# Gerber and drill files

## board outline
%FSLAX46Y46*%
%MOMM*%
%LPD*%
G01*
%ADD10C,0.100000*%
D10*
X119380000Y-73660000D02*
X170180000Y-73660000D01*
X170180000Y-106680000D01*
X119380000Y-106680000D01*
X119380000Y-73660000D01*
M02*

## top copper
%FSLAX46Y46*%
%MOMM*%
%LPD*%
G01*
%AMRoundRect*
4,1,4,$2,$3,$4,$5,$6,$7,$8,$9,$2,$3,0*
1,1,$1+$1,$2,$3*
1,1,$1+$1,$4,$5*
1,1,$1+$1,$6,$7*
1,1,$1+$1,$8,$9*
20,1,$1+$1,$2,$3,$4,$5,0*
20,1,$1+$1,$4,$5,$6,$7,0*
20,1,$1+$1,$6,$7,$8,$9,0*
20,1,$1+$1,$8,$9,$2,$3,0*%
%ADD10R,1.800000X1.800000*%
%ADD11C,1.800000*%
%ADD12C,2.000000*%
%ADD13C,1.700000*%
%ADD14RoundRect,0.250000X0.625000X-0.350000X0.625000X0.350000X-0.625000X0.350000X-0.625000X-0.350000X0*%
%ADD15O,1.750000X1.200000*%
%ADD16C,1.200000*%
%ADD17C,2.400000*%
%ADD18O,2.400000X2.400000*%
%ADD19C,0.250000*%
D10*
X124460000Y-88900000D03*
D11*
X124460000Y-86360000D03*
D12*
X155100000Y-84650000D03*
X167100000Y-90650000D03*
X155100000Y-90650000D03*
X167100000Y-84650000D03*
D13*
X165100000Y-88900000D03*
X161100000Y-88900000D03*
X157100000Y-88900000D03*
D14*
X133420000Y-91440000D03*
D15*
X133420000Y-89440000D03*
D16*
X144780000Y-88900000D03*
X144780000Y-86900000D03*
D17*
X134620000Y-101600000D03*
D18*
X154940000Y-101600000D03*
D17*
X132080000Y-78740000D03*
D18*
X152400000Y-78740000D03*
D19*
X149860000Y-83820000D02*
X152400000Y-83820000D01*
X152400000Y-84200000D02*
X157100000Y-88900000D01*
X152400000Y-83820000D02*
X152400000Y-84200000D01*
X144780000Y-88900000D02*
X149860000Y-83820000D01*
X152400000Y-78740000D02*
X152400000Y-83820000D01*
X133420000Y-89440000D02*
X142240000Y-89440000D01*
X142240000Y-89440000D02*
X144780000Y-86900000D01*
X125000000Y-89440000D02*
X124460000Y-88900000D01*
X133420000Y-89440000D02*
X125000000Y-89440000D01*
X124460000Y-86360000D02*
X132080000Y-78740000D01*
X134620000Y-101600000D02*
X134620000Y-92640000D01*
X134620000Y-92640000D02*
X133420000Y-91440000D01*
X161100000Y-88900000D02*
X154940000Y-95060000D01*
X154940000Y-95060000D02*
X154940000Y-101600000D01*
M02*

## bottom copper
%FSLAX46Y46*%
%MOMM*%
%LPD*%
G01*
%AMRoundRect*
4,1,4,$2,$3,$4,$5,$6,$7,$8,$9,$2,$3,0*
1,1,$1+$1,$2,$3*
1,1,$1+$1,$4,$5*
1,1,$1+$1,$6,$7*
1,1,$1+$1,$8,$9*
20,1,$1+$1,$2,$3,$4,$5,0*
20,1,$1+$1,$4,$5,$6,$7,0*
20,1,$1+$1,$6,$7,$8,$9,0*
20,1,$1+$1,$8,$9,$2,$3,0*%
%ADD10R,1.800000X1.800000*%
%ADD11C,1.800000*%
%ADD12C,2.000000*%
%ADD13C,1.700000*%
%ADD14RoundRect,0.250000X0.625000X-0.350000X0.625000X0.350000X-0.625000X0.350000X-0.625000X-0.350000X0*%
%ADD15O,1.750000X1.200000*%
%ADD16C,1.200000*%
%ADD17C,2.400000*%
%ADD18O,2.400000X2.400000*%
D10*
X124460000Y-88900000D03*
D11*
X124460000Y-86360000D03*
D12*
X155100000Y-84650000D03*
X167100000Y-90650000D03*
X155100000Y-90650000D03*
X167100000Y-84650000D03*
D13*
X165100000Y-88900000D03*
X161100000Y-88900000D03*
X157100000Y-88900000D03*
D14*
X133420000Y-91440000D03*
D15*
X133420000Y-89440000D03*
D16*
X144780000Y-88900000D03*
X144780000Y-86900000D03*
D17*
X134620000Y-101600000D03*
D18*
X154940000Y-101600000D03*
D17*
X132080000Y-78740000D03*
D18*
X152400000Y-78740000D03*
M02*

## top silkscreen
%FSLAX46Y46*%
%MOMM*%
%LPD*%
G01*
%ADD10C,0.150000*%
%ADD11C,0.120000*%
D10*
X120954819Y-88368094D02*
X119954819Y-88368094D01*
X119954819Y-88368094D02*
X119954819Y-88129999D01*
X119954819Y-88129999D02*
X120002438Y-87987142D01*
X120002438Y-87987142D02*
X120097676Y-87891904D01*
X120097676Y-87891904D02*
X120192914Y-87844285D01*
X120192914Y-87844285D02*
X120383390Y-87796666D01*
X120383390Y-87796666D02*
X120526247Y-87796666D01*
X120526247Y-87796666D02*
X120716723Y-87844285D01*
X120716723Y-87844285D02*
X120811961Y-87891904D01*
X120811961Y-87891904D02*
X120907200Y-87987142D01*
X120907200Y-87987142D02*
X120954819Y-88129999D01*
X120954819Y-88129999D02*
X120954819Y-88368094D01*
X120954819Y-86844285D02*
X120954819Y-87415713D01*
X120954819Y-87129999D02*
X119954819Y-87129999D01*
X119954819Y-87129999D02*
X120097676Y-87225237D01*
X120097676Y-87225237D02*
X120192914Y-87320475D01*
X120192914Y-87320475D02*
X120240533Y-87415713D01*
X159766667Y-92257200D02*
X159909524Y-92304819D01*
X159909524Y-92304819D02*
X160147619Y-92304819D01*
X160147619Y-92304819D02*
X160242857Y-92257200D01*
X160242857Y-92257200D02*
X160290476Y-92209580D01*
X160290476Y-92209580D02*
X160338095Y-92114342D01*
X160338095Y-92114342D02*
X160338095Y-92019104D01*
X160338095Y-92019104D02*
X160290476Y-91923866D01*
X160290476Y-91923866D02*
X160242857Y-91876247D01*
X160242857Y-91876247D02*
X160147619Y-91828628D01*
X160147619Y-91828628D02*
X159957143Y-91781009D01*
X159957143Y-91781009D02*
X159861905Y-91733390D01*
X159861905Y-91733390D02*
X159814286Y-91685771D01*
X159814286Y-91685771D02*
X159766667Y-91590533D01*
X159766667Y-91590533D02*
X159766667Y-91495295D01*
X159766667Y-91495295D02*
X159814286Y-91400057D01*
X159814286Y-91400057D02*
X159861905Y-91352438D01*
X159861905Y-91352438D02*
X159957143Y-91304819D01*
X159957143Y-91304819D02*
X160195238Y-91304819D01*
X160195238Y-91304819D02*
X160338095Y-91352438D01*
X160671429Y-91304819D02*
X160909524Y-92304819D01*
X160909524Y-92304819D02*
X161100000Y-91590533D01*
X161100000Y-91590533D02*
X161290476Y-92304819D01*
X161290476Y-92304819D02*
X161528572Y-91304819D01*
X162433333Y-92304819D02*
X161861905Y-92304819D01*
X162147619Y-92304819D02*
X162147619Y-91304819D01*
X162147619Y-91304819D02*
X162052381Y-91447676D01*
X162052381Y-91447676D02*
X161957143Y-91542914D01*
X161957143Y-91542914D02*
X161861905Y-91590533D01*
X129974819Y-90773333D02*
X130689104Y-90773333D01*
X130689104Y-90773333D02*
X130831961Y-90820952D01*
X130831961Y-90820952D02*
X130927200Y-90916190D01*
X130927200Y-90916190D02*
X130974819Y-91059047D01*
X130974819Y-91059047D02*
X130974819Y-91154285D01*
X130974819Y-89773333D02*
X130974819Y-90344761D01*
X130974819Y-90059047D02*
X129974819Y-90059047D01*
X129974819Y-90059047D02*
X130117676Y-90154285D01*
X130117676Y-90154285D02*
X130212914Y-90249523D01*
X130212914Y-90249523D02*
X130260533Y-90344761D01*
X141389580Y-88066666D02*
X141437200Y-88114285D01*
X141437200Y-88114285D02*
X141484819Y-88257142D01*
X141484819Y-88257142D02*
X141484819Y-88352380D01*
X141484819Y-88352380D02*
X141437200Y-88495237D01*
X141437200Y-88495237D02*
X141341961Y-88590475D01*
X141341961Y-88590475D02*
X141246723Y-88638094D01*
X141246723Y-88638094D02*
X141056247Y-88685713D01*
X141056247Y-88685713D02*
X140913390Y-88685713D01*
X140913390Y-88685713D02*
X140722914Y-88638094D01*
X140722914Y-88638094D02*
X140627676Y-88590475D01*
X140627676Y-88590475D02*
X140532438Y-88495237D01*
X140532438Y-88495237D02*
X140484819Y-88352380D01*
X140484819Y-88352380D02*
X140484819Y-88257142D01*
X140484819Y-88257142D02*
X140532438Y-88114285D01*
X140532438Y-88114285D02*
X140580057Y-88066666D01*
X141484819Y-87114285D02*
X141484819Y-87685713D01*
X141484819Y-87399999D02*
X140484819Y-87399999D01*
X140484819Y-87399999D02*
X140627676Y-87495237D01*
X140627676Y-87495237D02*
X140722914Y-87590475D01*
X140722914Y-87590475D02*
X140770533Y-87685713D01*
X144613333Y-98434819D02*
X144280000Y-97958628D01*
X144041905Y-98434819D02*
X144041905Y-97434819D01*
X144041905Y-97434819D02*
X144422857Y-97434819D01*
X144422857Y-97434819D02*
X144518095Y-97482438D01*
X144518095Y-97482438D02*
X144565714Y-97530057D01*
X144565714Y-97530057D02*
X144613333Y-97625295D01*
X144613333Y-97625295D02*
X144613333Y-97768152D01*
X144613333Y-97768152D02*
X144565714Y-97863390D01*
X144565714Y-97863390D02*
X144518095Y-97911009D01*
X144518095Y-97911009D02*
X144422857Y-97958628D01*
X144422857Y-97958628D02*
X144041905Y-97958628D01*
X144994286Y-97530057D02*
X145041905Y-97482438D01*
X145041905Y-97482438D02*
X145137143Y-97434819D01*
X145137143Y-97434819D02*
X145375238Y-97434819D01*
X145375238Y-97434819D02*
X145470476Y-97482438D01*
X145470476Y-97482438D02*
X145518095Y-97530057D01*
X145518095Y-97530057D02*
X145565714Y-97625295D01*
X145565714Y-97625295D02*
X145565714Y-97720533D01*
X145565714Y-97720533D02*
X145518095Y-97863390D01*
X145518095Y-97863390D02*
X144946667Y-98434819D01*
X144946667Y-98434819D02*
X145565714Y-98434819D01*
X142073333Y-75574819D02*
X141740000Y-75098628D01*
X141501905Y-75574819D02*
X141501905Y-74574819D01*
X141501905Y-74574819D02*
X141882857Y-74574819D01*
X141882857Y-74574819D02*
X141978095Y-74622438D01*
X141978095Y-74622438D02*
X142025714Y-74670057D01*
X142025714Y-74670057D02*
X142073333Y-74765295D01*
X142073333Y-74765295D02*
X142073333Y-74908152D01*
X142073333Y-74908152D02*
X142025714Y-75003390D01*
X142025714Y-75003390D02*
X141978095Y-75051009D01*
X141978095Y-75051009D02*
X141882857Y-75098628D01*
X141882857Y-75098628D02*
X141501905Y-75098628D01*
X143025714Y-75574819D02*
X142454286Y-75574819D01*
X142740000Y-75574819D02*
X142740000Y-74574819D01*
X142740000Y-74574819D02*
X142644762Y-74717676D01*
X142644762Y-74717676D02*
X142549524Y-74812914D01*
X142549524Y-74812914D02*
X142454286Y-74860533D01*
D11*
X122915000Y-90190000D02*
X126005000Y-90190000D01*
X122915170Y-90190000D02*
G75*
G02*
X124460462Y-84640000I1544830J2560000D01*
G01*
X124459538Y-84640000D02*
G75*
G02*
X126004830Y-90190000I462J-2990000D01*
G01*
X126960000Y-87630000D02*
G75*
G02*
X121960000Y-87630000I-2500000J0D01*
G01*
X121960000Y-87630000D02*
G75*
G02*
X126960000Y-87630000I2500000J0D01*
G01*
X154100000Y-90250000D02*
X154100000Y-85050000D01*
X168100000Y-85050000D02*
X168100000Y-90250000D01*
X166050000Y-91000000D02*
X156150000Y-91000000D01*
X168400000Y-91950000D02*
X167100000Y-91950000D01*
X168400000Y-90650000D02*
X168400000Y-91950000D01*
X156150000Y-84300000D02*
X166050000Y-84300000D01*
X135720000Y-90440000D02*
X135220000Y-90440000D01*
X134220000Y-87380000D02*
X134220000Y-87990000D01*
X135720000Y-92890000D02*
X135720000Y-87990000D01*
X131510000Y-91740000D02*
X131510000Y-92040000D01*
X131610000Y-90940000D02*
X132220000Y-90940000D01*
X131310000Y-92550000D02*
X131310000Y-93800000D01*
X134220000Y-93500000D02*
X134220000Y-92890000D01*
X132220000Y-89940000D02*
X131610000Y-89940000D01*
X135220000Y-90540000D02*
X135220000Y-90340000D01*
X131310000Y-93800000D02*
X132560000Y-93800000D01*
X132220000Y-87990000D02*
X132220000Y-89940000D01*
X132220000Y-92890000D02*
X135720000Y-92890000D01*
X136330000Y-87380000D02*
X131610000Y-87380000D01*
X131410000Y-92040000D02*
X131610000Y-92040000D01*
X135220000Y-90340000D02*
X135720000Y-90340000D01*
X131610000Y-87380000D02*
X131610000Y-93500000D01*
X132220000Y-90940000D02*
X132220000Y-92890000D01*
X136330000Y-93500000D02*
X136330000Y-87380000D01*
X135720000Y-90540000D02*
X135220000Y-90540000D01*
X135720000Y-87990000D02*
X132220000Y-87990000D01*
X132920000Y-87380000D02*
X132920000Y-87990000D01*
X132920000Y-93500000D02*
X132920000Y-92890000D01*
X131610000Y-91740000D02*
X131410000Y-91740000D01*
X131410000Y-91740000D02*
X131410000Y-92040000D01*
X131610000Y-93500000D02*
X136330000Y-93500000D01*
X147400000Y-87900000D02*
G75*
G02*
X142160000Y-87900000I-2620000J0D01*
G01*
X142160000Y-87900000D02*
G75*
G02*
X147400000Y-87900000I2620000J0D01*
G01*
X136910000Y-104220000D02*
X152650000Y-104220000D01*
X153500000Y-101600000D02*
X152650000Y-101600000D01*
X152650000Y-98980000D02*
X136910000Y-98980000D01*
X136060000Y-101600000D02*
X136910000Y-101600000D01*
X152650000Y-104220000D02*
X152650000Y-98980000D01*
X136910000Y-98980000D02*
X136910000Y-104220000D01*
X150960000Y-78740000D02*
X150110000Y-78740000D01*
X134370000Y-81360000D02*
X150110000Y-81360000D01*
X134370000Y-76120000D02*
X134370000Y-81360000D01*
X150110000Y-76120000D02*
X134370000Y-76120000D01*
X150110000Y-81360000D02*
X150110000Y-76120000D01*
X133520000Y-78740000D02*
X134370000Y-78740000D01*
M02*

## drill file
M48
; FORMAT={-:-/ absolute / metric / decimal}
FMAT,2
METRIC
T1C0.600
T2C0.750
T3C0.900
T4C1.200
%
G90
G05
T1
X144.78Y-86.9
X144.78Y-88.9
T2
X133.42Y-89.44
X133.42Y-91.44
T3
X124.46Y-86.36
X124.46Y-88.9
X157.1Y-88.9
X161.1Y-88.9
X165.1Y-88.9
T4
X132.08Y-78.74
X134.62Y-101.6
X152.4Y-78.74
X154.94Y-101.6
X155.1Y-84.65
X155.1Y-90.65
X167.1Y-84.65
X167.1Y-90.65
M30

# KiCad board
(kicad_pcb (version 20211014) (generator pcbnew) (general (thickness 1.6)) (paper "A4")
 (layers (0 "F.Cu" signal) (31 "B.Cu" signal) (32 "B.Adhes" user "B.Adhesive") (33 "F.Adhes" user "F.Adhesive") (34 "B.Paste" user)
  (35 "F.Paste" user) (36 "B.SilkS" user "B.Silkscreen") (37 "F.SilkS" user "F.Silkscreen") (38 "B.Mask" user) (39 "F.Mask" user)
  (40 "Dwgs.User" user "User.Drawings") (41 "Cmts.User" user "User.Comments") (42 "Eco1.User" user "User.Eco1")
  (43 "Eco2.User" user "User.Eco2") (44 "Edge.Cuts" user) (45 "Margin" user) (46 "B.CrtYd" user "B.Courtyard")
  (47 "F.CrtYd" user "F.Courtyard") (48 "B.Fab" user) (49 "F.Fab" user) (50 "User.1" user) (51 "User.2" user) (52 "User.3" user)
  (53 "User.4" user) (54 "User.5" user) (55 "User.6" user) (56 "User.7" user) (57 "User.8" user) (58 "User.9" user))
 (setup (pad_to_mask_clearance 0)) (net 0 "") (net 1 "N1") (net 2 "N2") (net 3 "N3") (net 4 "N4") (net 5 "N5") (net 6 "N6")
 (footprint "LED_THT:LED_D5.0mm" (layer "F.Cu") (at 124.46 88.9 90)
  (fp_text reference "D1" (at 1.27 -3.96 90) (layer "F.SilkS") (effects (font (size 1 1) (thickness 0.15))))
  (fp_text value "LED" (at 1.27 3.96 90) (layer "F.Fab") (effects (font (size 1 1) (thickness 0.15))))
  (fp_line (start -1.29 -1.545) (end -1.29 1.545) (layer "F.SilkS") (width 0.12))
  (fp_arc (start -1.29 -1.54483) (mid 2.072002 -2.880433) (end 4.26 0.000462) (layer "F.SilkS") (width 0.12))
  (fp_arc (start 4.26 -0.000462) (mid 2.072002 2.880433) (end -1.29 1.54483) (layer "F.SilkS") (width 0.12))
  (fp_circle (center 1.27 0) (end 3.77 0) (layer "F.SilkS") (width 0.12) (fill none))
  (pad "1" thru_hole rect (at 0 0 90) (size 1.8 1.8) (drill 0.9) (layers *.Cu *.Mask) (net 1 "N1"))
  (pad "2" thru_hole circle (at 2.54 0 90) (size 1.8 1.8) (drill 0.9) (layers *.Cu *.Mask) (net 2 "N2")))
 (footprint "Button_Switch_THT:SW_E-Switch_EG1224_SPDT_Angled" (layer "F.Cu") (at 165.1 88.9 180)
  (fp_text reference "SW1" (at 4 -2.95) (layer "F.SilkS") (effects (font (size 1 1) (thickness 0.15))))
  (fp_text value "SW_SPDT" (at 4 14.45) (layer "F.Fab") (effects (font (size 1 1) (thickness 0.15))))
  (fp_line (start 11 -1.35) (end 11 3.85) (layer "F.SilkS") (width 0.12))
  (fp_line (start -3 3.85) (end -3 -1.35) (layer "F.SilkS") (width 0.12))
  (fp_line (start -0.95 -2.1) (end 8.95 -2.1) (layer "F.SilkS") (width 0.12))
  (fp_line (start -3.3 -3.05) (end -2 -3.05) (layer "F.SilkS") (width 0.12))
  (fp_line (start -3.3 -1.75) (end -3.3 -3.05) (layer "F.SilkS") (width 0.12))
  (fp_line (start 8.95 4.6) (end -0.95 4.6) (layer "F.SilkS") (width 0.12))
  (pad "" thru_hole circle (at 10 4.25 180) (size 2 2) (drill 1.2) (layers *.Cu *.Mask))
  (pad "" thru_hole circle (at -2 -1.75 180) (size 2 2) (drill 1.2) (layers *.Cu *.Mask))
  (pad "" thru_hole circle (at 10 -1.75 180) (size 2 2) (drill 1.2) (layers *.Cu *.Mask))
  (pad "" thru_hole circle (at -2 4.25 180) (size 2 2) (drill 1.2) (layers *.Cu *.Mask))
  (pad "1" thru_hole circle (at 0 0 180) (size 1.7 1.7) (drill 0.9) (layers *.Cu *.Mask) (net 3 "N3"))
  (pad "2" thru_hole circle (at 4 0 180) (size 1.7 1.7) (drill 0.9) (layers *.Cu *.Mask) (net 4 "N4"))
  (pad "3" thru_hole circle (at 8 0 180) (size 1.7 1.7) (drill 0.9) (layers *.Cu *.Mask) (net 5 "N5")))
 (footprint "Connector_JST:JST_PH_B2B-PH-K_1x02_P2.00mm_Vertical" (layer "F.Cu") (at 133.42 91.44 90)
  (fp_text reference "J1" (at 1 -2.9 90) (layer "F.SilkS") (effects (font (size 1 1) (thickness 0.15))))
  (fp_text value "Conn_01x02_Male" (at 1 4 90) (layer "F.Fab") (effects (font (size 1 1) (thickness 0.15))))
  (fp_line (start 1 2.3) (end 1 1.8) (layer "F.SilkS") (width 0.12))
  (fp_line (start 4.06 0.8) (end 3.45 0.8) (layer "F.SilkS") (width 0.12))
  (fp_line (start -1.45 2.3) (end 3.45 2.3) (layer "F.SilkS") (width 0.12))
  (fp_line (start -0.3 -1.91) (end -0.6 -1.91) (layer "F.SilkS") (width 0.12))
  (fp_line (start 0.5 -1.81) (end 0.5 -1.2) (layer "F.SilkS") (width 0.12))
  (fp_line (start -1.11 -2.11) (end -2.36 -2.11) (layer "F.SilkS") (width 0.12))
  (fp_line (start -2.06 0.8) (end -1.45 0.8) (layer "F.SilkS") (width 0.12))
  (fp_line (start 1.5 -1.2) (end 1.5 -1.81) (layer "F.SilkS") (width 0.12))
  (fp_line (start 0.9 1.8) (end 1.1 1.8) (layer "F.SilkS") (width 0.12))
  (fp_line (start -2.36 -2.11) (end -2.36 -0.86) (layer "F.SilkS") (width 0.12))
  (fp_line (start 3.45 -1.2) (end 1.5 -1.2) (layer "F.SilkS") (width 0.12))
  (fp_line (start -1.45 -1.2) (end -1.45 2.3) (layer "F.SilkS") (width 0.12))
  (fp_line (start 4.06 2.91) (end 4.06 -1.81) (layer "F.SilkS") (width 0.12))
  (fp_line (start -0.6 -2.01) (end -0.6 -1.81) (layer "F.SilkS") (width 0.12))
  (fp_line (start 1.1 1.8) (end 1.1 2.3) (layer "F.SilkS") (width 0.12))
  (fp_line (start 4.06 -1.81) (end -2.06 -1.81) (layer "F.SilkS") (width 0.12))
  (fp_line (start 0.5 -1.2) (end -1.45 -1.2) (layer "F.SilkS") (width 0.12))
  (fp_line (start -2.06 2.91) (end 4.06 2.91) (layer "F.SilkS") (width 0.12))
  (fp_line (start 0.9 2.3) (end 0.9 1.8) (layer "F.SilkS") (width 0.12))
  (fp_line (start 3.45 2.3) (end 3.45 -1.2) (layer "F.SilkS") (width 0.12))
  (fp_line (start 4.06 -0.5) (end 3.45 -0.5) (layer "F.SilkS") (width 0.12))
  (fp_line (start -2.06 -0.5) (end -1.45 -0.5) (layer "F.SilkS") (width 0.12))
  (fp_line (start -0.3 -1.81) (end -0.3 -2.01) (layer "F.SilkS") (width 0.12))
  (fp_line (start -0.3 -2.01) (end -0.6 -2.01) (layer "F.SilkS") (width 0.12))
  (fp_line (start -2.06 -1.81) (end -2.06 2.91) (layer "F.SilkS") (width 0.12))
  (pad "1" thru_hole roundrect (at 0 0 90) (size 1.2 1.75) (drill 0.75) (layers *.Cu *.Mask) (roundrect_rratio 0.208333) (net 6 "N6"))
  (pad "2" thru_hole oval (at 2 0 90) (size 1.2 1.75) (drill 0.75) (layers *.Cu *.Mask) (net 1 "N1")))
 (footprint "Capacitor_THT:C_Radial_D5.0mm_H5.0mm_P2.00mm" (layer "F.Cu") (at 144.78 88.9 90)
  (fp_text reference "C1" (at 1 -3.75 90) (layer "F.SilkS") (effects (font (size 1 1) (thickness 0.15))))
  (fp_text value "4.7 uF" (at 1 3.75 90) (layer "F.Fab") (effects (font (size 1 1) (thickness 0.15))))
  (fp_circle (center 1 0) (end 3.62 0) (layer "F.SilkS") (width 0.12) (fill none))
  (pad "1" thru_hole circle (at 0 0 90) (size 1.2 1.2) (drill 0.6) (layers *.Cu *.Mask) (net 5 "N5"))
  (pad "2" thru_hole circle (at 2 0 90) (size 1.2 1.2) (drill 0.6) (layers *.Cu *.Mask) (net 1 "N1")))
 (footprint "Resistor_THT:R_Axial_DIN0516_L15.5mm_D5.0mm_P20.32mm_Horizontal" (layer "F.Cu") (at 134.62 101.6)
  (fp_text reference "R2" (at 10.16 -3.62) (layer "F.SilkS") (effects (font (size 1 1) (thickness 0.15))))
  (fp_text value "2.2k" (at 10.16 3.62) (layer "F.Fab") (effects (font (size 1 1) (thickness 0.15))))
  (fp_line (start 2.29 2.62) (end 18.03 2.62) (layer "F.SilkS") (width 0.12))
  (fp_line (start 18.88 0) (end 18.03 0) (layer "F.SilkS") (width 0.12))
  (fp_line (start 18.03 -2.62) (end 2.29 -2.62) (layer "F.SilkS") (width 0.12))
  (fp_line (start 1.44 0) (end 2.29 0) (layer "F.SilkS") (width 0.12))
  (fp_line (start 18.03 2.62) (end 18.03 -2.62) (layer "F.SilkS") (width 0.12))
  (fp_line (start 2.29 -2.62) (end 2.29 2.62) (layer "F.SilkS") (width 0.12))
  (pad "1" thru_hole circle (at 0 0) (size 2.4 2.4) (drill 1.2) (layers *.Cu *.Mask) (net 6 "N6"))
  (pad "2" thru_hole oval (at 20.32 0) (size 2.4 2.4) (drill 1.2) (layers *.Cu *.Mask) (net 4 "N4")))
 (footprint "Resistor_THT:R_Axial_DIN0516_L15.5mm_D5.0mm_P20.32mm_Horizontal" (layer "F.Cu") (at 132.08 78.74)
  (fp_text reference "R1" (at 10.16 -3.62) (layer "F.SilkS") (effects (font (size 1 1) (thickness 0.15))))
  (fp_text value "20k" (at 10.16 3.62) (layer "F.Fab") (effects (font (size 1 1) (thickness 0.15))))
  (fp_line (start 18.88 0) (end 18.03 0) (layer "F.SilkS") (width 0.12))
  (fp_line (start 2.29 2.62) (end 18.03 2.62) (layer "F.SilkS") (width 0.12))
  (fp_line (start 2.29 -2.62) (end 2.29 2.62) (layer "F.SilkS") (width 0.12))
  (fp_line (start 18.03 -2.62) (end 2.29 -2.62) (layer "F.SilkS") (width 0.12))
  (fp_line (start 18.03 2.62) (end 18.03 -2.62) (layer "F.SilkS") (width 0.12))
  (fp_line (start 1.44 0) (end 2.29 0) (layer "F.SilkS") (width 0.12))
  (pad "1" thru_hole circle (at 0 0) (size 2.4 2.4) (drill 1.2) (layers *.Cu *.Mask) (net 2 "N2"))
  (pad "2" thru_hole oval (at 20.32 0) (size 2.4 2.4) (drill 1.2) (layers *.Cu *.Mask) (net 5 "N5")))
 (gr_rect (start 119.38 73.66) (end 170.18 106.68) (layer "Edge.Cuts") (width 0.1) (fill none))
 (segment (start 149.86 83.82) (end 152.4 83.82) (width 0.25) (layer "F.Cu") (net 5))
 (segment (start 152.4 84.2) (end 157.1 88.9) (width 0.25) (layer "F.Cu") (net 5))
 (segment (start 152.4 83.82) (end 152.4 84.2) (width 0.25) (layer "F.Cu") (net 5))
 (segment (start 144.78 88.9) (end 149.86 83.82) (width 0.25) (layer "F.Cu") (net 5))
 (segment (start 152.4 78.74) (end 152.4 83.82) (width 0.25) (layer "F.Cu") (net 5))
 (segment (start 133.42 89.44) (end 142.24 89.44) (width 0.25) (layer "F.Cu") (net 1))
 (segment (start 142.24 89.44) (end 144.78 86.9) (width 0.25) (layer "F.Cu") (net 1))
 (segment (start 125 89.44) (end 124.46 88.9) (width 0.25) (layer "F.Cu") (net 1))
 (segment (start 133.42 89.44) (end 125 89.44) (width 0.25) (layer "F.Cu") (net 1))
 (segment (start 124.46 86.36) (end 132.08 78.74) (width 0.25) (layer "F.Cu") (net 2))
 (segment (start 134.62 101.6) (end 134.62 92.64) (width 0.25) (layer "F.Cu") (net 6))
 (segment (start 134.62 92.64) (end 133.42 91.44) (width 0.25) (layer "F.Cu") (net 6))
 (segment (start 161.1 88.9) (end 154.94 95.06) (width 0.25) (layer "F.Cu") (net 4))
 (segment (start 154.94 95.06) (end 154.94 101.6) (width 0.25) (layer "F.Cu") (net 4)))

